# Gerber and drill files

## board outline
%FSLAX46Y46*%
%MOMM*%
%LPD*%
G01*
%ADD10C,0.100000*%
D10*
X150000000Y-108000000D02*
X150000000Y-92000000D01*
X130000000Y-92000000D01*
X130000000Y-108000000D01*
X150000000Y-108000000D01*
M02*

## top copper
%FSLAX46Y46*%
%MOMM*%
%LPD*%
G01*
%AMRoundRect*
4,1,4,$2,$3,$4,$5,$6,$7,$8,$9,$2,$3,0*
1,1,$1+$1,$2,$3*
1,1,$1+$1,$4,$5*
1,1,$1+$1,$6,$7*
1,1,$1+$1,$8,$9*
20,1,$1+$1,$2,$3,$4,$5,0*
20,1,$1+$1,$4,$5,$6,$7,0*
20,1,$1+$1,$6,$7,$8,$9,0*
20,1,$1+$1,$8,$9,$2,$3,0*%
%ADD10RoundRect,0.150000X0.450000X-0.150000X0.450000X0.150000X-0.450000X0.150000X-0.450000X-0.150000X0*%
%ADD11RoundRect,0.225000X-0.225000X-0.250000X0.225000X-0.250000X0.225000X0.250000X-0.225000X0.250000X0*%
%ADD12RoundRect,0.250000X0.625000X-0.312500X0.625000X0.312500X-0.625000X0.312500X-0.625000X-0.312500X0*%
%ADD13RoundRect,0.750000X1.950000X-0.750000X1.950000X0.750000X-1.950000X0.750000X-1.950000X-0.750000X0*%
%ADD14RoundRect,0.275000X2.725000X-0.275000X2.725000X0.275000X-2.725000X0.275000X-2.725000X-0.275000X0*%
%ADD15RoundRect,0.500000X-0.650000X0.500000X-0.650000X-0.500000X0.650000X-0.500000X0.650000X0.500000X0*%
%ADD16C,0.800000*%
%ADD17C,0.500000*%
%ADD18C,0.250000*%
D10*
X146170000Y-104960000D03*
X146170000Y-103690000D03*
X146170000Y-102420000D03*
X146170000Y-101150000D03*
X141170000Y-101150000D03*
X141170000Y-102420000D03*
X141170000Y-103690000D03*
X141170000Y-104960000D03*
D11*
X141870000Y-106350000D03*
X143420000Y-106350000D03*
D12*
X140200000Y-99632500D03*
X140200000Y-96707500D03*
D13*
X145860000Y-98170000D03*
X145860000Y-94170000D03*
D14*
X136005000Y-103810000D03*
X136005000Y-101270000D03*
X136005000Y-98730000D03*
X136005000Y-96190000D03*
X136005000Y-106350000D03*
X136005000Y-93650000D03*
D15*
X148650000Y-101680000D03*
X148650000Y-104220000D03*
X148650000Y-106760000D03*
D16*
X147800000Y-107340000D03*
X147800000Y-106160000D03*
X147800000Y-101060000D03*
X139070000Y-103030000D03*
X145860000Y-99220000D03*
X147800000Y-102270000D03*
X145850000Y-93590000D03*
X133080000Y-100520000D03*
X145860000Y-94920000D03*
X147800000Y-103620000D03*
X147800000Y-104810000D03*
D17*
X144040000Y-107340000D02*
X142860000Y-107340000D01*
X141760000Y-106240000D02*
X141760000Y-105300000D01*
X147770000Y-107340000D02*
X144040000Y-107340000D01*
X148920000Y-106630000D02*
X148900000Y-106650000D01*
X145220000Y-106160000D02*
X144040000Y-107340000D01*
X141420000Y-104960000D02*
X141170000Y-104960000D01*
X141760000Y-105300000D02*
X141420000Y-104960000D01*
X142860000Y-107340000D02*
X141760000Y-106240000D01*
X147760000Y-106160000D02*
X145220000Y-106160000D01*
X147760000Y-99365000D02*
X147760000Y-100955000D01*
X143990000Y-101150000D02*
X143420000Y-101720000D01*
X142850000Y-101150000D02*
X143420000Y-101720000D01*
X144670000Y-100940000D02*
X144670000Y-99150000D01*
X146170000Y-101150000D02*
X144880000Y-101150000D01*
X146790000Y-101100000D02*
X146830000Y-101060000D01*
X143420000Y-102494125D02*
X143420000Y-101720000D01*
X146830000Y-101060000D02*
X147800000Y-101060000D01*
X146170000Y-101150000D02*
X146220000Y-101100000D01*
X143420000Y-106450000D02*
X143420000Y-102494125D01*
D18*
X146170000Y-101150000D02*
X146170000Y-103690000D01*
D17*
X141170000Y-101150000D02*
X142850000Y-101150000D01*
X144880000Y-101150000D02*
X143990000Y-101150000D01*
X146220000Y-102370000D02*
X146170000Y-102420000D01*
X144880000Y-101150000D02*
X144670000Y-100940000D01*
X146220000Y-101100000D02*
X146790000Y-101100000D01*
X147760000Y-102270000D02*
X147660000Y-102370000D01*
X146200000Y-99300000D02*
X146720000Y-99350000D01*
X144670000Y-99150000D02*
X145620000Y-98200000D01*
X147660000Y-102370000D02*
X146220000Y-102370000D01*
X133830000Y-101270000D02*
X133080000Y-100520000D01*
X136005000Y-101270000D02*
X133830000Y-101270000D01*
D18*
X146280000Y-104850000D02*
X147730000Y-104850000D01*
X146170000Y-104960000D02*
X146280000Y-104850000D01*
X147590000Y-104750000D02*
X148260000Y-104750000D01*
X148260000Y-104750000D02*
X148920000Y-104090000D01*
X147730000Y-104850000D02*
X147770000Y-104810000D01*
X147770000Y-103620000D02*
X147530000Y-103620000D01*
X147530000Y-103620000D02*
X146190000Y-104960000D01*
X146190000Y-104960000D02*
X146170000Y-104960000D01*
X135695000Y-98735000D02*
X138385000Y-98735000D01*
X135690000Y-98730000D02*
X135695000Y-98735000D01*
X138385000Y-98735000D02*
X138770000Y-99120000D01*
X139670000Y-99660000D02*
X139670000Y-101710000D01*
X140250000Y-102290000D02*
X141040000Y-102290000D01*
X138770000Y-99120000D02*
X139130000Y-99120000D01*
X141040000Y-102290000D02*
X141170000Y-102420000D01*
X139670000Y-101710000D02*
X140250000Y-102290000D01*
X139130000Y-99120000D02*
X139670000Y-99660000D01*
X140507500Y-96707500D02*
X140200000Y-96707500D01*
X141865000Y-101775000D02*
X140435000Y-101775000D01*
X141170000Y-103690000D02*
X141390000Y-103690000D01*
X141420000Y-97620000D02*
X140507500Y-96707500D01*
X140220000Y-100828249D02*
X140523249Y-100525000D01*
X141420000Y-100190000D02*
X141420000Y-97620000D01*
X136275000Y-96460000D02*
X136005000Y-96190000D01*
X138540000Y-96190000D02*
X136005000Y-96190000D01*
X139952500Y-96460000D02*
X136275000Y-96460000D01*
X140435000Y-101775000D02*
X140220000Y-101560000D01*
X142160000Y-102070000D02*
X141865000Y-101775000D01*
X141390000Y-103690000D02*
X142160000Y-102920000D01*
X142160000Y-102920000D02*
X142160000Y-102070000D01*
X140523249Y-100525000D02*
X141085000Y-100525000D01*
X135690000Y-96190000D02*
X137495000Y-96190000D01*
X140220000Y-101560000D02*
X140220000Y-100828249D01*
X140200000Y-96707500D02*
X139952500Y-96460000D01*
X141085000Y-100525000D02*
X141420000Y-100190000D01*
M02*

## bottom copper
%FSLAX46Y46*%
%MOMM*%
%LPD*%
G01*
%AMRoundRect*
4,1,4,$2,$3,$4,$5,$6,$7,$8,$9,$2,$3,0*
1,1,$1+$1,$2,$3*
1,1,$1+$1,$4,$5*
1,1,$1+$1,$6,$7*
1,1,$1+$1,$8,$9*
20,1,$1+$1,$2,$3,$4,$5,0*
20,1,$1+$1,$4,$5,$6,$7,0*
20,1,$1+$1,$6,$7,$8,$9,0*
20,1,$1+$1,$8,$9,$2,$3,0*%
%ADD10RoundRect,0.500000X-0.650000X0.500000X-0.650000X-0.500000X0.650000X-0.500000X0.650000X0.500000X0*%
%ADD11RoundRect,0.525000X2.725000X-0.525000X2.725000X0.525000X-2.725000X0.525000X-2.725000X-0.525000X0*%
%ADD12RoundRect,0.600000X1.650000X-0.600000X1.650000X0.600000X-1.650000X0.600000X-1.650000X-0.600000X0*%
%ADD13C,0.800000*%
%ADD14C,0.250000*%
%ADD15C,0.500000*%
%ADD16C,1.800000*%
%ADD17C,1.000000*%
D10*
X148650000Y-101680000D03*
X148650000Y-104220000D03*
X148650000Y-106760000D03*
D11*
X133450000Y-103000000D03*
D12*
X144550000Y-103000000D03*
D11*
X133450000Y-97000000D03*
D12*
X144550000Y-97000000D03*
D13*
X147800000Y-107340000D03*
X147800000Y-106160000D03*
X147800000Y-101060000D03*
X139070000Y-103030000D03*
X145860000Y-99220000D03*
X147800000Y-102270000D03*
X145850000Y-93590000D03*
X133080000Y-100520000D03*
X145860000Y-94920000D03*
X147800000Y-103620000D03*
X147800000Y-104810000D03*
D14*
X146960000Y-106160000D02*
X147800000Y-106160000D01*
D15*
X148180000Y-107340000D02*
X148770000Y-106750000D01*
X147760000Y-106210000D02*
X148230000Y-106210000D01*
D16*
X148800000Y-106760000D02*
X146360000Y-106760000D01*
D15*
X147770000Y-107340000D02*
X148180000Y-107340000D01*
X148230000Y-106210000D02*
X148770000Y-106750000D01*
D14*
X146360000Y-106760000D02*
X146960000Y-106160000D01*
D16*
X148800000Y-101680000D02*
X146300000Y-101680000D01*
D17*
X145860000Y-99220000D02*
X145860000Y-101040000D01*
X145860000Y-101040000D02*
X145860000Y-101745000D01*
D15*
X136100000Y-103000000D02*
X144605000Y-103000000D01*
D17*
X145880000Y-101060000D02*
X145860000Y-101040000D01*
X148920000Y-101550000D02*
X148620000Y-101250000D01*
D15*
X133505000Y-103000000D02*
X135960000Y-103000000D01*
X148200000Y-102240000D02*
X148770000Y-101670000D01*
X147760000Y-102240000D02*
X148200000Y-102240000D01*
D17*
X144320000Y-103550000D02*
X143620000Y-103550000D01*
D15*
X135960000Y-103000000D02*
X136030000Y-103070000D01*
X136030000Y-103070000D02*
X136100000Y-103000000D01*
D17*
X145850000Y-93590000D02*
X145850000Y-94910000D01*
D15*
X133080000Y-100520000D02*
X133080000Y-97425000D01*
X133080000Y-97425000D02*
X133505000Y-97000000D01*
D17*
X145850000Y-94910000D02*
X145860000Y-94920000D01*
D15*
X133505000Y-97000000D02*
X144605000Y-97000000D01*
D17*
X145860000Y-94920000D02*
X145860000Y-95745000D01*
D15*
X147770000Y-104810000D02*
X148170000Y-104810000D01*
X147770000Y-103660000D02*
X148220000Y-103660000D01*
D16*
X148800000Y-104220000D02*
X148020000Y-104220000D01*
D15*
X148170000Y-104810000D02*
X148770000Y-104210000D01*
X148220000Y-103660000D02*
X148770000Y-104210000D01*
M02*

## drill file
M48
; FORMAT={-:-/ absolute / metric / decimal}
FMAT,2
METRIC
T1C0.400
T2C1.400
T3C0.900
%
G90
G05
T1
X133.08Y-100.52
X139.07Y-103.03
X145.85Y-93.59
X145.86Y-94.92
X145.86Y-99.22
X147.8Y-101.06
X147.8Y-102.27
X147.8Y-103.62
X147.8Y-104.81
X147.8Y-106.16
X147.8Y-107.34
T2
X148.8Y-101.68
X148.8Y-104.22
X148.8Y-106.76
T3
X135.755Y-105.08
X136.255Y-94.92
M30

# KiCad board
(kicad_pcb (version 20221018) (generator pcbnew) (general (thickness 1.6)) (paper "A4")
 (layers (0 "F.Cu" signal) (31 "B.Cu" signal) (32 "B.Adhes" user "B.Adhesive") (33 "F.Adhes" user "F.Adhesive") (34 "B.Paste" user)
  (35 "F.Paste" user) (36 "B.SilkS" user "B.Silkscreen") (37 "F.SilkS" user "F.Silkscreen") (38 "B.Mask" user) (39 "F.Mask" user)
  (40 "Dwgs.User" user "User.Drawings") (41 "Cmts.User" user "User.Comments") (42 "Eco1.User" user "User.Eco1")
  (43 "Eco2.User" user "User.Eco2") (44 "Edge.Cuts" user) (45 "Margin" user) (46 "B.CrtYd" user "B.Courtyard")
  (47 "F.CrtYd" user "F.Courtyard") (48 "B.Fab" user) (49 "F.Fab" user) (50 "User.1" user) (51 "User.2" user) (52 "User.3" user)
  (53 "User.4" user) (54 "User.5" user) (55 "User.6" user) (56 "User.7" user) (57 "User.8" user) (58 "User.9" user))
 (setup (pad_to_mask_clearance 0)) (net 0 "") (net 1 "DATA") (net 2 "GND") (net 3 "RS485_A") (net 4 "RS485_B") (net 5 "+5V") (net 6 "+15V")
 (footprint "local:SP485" (layer "F.Cu") (at 143.67 103.055 90)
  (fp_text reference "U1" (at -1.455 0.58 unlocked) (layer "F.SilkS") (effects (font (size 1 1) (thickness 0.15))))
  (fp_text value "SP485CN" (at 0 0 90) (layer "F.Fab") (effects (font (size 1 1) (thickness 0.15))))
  (pad "1" smd roundrect (at -1.905 2.5 90) (size 0.6 1.2) (layers "F.Cu" "F.Paste" "F.Mask") (roundrect_rratio 0.25) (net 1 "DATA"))
  (pad "2" smd roundrect (at -0.635 2.5 90) (size 0.6 1.2) (layers "F.Cu" "F.Paste" "F.Mask") (roundrect_rratio 0.25) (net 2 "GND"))
  (pad "3" smd roundrect (at 0.635 2.5 90) (size 0.6 1.2) (layers "F.Cu" "F.Paste" "F.Mask") (roundrect_rratio 0.25) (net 2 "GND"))
  (pad "4" smd roundrect (at 1.905 2.5 90) (size 0.6 1.2) (layers "F.Cu" "F.Paste" "F.Mask") (roundrect_rratio 0.25) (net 2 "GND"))
  (pad "5" smd roundrect (at 1.905 -2.5 90) (size 0.6 1.2) (layers "F.Cu" "F.Paste" "F.Mask") (roundrect_rratio 0.25) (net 2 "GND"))
  (pad "6" smd roundrect (at 0.635 -2.5 90) (size 0.6 1.2) (layers "F.Cu" "F.Paste" "F.Mask") (roundrect_rratio 0.25) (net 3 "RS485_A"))
  (pad "7" smd roundrect (at -0.635 -2.5 90) (size 0.6 1.2) (layers "F.Cu" "F.Paste" "F.Mask") (roundrect_rratio 0.25) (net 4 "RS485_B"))
  (pad "8" smd roundrect (at -1.905 -2.5 90) (size 0.6 1.2) (layers "F.Cu" "F.Paste" "F.Mask") (roundrect_rratio 0.25) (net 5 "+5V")))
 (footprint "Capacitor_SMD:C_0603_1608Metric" (layer "F.Cu") (at 142.645 106.35)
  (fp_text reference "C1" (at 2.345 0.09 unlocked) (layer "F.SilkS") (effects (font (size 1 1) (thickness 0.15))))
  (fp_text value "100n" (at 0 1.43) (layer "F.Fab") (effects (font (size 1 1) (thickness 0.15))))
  (pad "1" smd roundrect (at -0.775 0) (size 0.9 0.95) (layers "F.Cu" "F.Paste" "F.Mask") (roundrect_rratio 0.25) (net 5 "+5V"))
  (pad "2" smd roundrect (at 0.775 0) (size 0.9 0.95) (layers "F.Cu" "F.Paste" "F.Mask") (roundrect_rratio 0.25) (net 2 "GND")))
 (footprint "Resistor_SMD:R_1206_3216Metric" (layer "F.Cu") (at 140.2 98.17 90)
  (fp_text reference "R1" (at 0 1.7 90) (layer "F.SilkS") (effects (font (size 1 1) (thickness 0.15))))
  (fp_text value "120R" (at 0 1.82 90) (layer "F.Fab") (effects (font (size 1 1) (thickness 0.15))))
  (pad "1" smd roundrect (at -1.4625 0 90) (size 1.125 1.75) (layers "F.Cu" "F.Paste" "F.Mask") (roundrect_rratio 0.222222)
   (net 3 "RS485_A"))
  (pad "2" smd roundrect (at 1.4625 0 90) (size 1.125 1.75) (layers "F.Cu" "F.Paste" "F.Mask") (roundrect_rratio 0.222222) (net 4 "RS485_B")))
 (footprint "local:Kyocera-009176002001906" (layer "F.Cu") (at 145.86 96.17 90)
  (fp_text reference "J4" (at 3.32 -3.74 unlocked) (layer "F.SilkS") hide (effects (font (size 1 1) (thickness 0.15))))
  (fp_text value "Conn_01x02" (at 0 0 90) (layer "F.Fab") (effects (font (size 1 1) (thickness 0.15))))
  (pad "1" smd roundrect (at -2 0 90) (size 3 5.4) (layers "F.Cu" "F.Paste" "F.Mask") (roundrect_rratio 0.25) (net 2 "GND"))
  (pad "2" smd roundrect (at 2 0 90) (size 3 5.4) (layers "F.Cu" "F.Paste" "F.Mask") (roundrect_rratio 0.25) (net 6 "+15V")))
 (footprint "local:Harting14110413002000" (layer "F.Cu") (at 136.005 100 90)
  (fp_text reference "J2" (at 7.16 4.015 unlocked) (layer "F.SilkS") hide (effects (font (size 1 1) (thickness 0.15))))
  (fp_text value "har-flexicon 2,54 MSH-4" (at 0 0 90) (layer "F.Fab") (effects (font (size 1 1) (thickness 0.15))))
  (pad "" np_thru_hole circle (at -5.08 -0.25 90) (size 0.9 0.9) (drill 0.9) (layers "*.Cu" "*.Mask"))
  (pad "" np_thru_hole circle (at 5.08 0.25 90) (size 0.9 0.9) (drill 0.9) (layers "*.Cu" "*.Mask"))
  (pad "1" smd roundrect (at -3.81 0 90) (size 1.1 6) (layers "F.Cu" "F.Paste" "F.Mask") (roundrect_rratio 0.25) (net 2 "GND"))
  (pad "2" smd roundrect (at -1.27 0 90) (size 1.1 6) (layers "F.Cu" "F.Paste" "F.Mask") (roundrect_rratio 0.25) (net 6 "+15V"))
  (pad "3" smd roundrect (at 1.27 0 90) (size 1.1 6) (layers "F.Cu" "F.Paste" "F.Mask") (roundrect_rratio 0.25) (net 3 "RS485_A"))
  (pad "4" smd roundrect (at 3.81 0 90) (size 1.1 6) (layers "F.Cu" "F.Paste" "F.Mask") (roundrect_rratio 0.25) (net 4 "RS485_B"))
  (pad "MP1" smd roundrect (at -6.35 0 90) (size 1.1 6) (layers "F.Cu" "F.Paste" "F.Mask") (roundrect_rratio 0.25))
  (pad "MP2" smd roundrect (at 6.35 0 90) (size 1.1 6) (layers "F.Cu" "F.Paste" "F.Mask") (roundrect_rratio 0.25)))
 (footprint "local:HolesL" (layer "F.Cu") (at 148.8 104.22 -90)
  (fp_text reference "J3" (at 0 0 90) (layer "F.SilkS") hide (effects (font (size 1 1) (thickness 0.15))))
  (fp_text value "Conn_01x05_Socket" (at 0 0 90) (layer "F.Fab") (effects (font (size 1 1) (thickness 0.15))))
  (pad "1" thru_hole roundrect (at -2.54 0 270) (size 2 2.3) (drill 1.4 (offset 0 0.15)) (layers "*.Cu" "*.Mask") (roundrect_rratio 0.25)
   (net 2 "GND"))
  (pad "2" thru_hole roundrect (at 0 0 270) (size 2 2.3) (drill 1.4 (offset 0 0.15)) (layers "*.Cu" "*.Mask") (roundrect_rratio 0.25)
   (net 1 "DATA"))
  (pad "3" thru_hole roundrect (at 2.54 0 270) (size 2 2.3) (drill 1.4 (offset 0 0.15)) (layers "*.Cu" "*.Mask") (roundrect_rratio 0.25)
   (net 5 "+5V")))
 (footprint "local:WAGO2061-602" (layer "B.Cu") (at 138.2 100 90)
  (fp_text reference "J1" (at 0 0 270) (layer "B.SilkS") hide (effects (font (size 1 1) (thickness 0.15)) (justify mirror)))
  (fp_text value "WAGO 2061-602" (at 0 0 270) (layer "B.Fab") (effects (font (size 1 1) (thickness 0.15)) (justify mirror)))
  (pad "1" smd roundrect (at -3 -4.75 90) (size 2.1 6.5) (layers "B.Cu" "B.Paste" "B.Mask") (roundrect_rratio 0.25) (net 2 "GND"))
  (pad "1" smd roundrect (at -3 6.35 90) (size 2.4 4.5) (layers "B.Cu" "B.Paste" "B.Mask") (roundrect_rratio 0.25) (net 2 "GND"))
  (pad "2" smd roundrect (at 3 -4.75 90) (size 2.1 6.5) (layers "B.Cu" "B.Paste" "B.Mask") (roundrect_rratio 0.25) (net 6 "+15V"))
  (pad "2" smd roundrect (at 3 6.35 90) (size 2.4 4.5) (layers "B.Cu" "B.Paste" "B.Mask") (roundrect_rratio 0.25) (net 6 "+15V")))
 (gr_poly (pts (xy 150 108) (xy 150 92) (xy 130 92) (xy 130 108)) (stroke (width 0.1) (type solid)) (fill none) (layer "Edge.Cuts"))
 (segment (start 144.04 107.34) (end 142.86 107.34) (width 0.5) (layer "F.Cu") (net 5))
 (segment (start 141.76 106.24) (end 141.76 105.3) (width 0.5) (layer "F.Cu") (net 5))
 (segment (start 147.77 107.34) (end 144.04 107.34) (width 0.5) (layer "F.Cu") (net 5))
 (segment (start 148.92 106.63) (end 148.9 106.65) (width 0.5) (layer "F.Cu") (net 5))
 (segment (start 145.22 106.16) (end 144.04 107.34) (width 0.5) (layer "F.Cu") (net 5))
 (segment (start 141.42 104.96) (end 141.17 104.96) (width 0.5) (layer "F.Cu") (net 5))
 (segment (start 141.76 105.3) (end 141.42 104.96) (width 0.5) (layer "F.Cu") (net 5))
 (segment (start 142.86 107.34) (end 141.76 106.24) (width 0.5) (layer "F.Cu") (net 5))
 (segment (start 147.76 106.16) (end 145.22 106.16) (width 0.5) (layer "F.Cu") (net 5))
 (via (at 147.8 107.34) (size 0.8) (drill 0.4) (layers "F.Cu" "B.Cu") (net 5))
 (via (at 147.8 106.16) (size 0.8) (drill 0.4) (layers "F.Cu" "B.Cu") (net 5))
 (segment (start 146.96 106.16) (end 147.8 106.16) (width 0.25) (layer "B.Cu") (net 5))
 (segment (start 148.18 107.34) (end 148.77 106.75) (width 0.5) (layer "B.Cu") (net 5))
 (segment (start 147.76 106.21) (end 148.23 106.21) (width 0.5) (layer "B.Cu") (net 5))
 (segment (start 148.8 106.76) (end 146.36 106.76) (width 1.8) (layer "B.Cu") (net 5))
 (segment (start 147.77 107.34) (end 148.18 107.34) (width 0.5) (layer "B.Cu") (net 5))
 (segment (start 148.23 106.21) (end 148.77 106.75) (width 0.5) (layer "B.Cu") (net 5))
 (segment (start 146.36 106.76) (end 146.96 106.16) (width 0.25) (layer "B.Cu") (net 5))
 (segment (start 147.76 99.365) (end 147.76 100.955) (width 0.5) (layer "F.Cu") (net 2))
 (segment (start 143.99 101.15) (end 143.42 101.72) (width 0.5) (layer "F.Cu") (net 2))
 (segment (start 142.85 101.15) (end 143.42 101.72) (width 0.5) (layer "F.Cu") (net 2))
 (segment (start 144.67 100.94) (end 144.67 99.15) (width 0.5) (layer "F.Cu") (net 2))
 (segment (start 146.17 101.15) (end 144.88 101.15) (width 0.5) (layer "F.Cu") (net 2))
 (segment (start 146.79 101.1) (end 146.83 101.06) (width 0.5) (layer "F.Cu") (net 2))
 (segment (start 143.42 102.494125) (end 143.42 101.72) (width 0.5) (layer "F.Cu") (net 2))
 (segment (start 146.83 101.06) (end 147.8 101.06) (width 0.5) (layer "F.Cu") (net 2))
 (segment (start 146.17 101.15) (end 146.22 101.1) (width 0.5) (layer "F.Cu") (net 2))
 (segment (start 143.42 106.45) (end 143.42 102.494125) (width 0.5) (layer "F.Cu") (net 2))
 (segment (start 146.17 101.15) (end 146.17 103.69) (width 0.25) (layer "F.Cu") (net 2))
 (segment (start 141.17 101.15) (end 142.85 101.15) (width 0.5) (layer "F.Cu") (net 2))
 (segment (start 144.88 101.15) (end 143.99 101.15) (width 0.5) (layer "F.Cu") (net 2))
 (segment (start 146.22 102.37) (end 146.17 102.42) (width 0.5) (layer "F.Cu") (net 2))
 (segment (start 144.88 101.15) (end 144.67 100.94) (width 0.5) (layer "F.Cu") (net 2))
 (segment (start 146.22 101.1) (end 146.79 101.1) (width 0.5) (layer "F.Cu") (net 2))
 (segment (start 147.76 102.27) (end 147.66 102.37) (width 0.5) (layer "F.Cu") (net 2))
 (segment (start 146.2 99.3) (end 146.72 99.35) (width 0.5) (layer "F.Cu") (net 2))
 (segment (start 144.67 99.15) (end 145.62 98.2) (width 0.5) (layer "F.Cu") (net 2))
 (segment (start 147.66 102.37) (end 146.22 102.37) (width 0.5) (layer "F.Cu") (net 2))
 (via (at 147.8 101.06) (size 0.8) (drill 0.4) (layers "F.Cu" "B.Cu") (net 2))
 (via (at 139.07 103.03) (size 0.8) (drill 0.4) (layers "F.Cu" "B.Cu") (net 2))
 (via (at 145.86 99.22) (size 0.8) (drill 0.4) (layers "F.Cu" "B.Cu") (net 2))
 (via (at 147.8 102.27) (size 0.8) (drill 0.4) (layers "F.Cu" "B.Cu") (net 2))
 (segment (start 148.8 101.68) (end 146.3 101.68) (width 1.8) (layer "B.Cu") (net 2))
 (segment (start 145.86 99.22) (end 145.86 101.04) (width 1) (layer "B.Cu") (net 2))
 (segment (start 145.86 101.04) (end 145.86 101.745) (width 1) (layer "B.Cu") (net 2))
 (segment (start 136.1 103) (end 144.605 103) (width 0.5) (layer "B.Cu") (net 2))
 (segment (start 145.88 101.06) (end 145.86 101.04) (width 1) (layer "B.Cu") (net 2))
 (segment (start 148.92 101.55) (end 148.62 101.25) (width 1) (layer "B.Cu") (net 2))
 (segment (start 133.505 103) (end 135.96 103) (width 0.5) (layer "B.Cu") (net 2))
 (segment (start 148.2 102.24) (end 148.77 101.67) (width 0.5) (layer "B.Cu") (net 2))
 (segment (start 147.76 102.24) (end 148.2 102.24) (width 0.5) (layer "B.Cu") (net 2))
 (segment (start 144.32 103.55) (end 143.62 103.55) (width 1) (layer "B.Cu") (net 2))
 (segment (start 135.96 103) (end 136.03 103.07) (width 0.5) (layer "B.Cu") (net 2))
 (segment (start 136.03 103.07) (end 136.1 103) (width 0.5) (layer "B.Cu") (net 2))
 (segment (start 133.83 101.27) (end 133.08 100.52) (width 0.5) (layer "F.Cu") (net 6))
 (segment (start 136.005 101.27) (end 133.83 101.27) (width 0.5) (layer "F.Cu") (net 6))
 (via (at 145.85 93.59) (size 0.8) (drill 0.4) (layers "F.Cu" "B.Cu") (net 6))
 (via (at 133.08 100.52) (size 0.8) (drill 0.4) (layers "F.Cu" "B.Cu") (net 6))
 (via (at 145.86 94.92) (size 0.8) (drill 0.4) (layers "F.Cu" "B.Cu") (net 6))
 (segment (start 145.85 93.59) (end 145.85 94.91) (width 1) (layer "B.Cu") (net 6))
 (segment (start 133.08 100.52) (end 133.08 97.425) (width 0.5) (layer "B.Cu") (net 6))
 (segment (start 133.08 97.425) (end 133.505 97) (width 0.5) (layer "B.Cu") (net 6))
 (segment (start 145.85 94.91) (end 145.86 94.92) (width 1) (layer "B.Cu") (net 6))
 (segment (start 133.505 97) (end 144.605 97) (width 0.5) (layer "B.Cu") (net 6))
 (segment (start 145.86 94.92) (end 145.86 95.745) (width 1) (layer "B.Cu") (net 6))
 (segment (start 146.28 104.85) (end 147.73 104.85) (width 0.25) (layer "F.Cu") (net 1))
 (segment (start 146.17 104.96) (end 146.28 104.85) (width 0.25) (layer "F.Cu") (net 1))
 (segment (start 147.59 104.75) (end 148.26 104.75) (width 0.25) (layer "F.Cu") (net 1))
 (segment (start 148.26 104.75) (end 148.92 104.09) (width 0.25) (layer "F.Cu") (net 1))
 (segment (start 147.73 104.85) (end 147.77 104.81) (width 0.25) (layer "F.Cu") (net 1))
 (segment (start 147.77 103.62) (end 147.53 103.62) (width 0.25) (layer "F.Cu") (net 1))
 (segment (start 147.53 103.62) (end 146.19 104.96) (width 0.25) (layer "F.Cu") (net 1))
 (segment (start 146.19 104.96) (end 146.17 104.96) (width 0.25) (layer "F.Cu") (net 1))
 (via (at 147.8 103.62) (size 0.8) (drill 0.4) (layers "F.Cu" "B.Cu") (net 1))
 (via (at 147.8 104.81) (size 0.8) (drill 0.4) (layers "F.Cu" "B.Cu") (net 1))
 (segment (start 147.77 104.81) (end 148.17 104.81) (width 0.5) (layer "B.Cu") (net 1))
 (segment (start 147.77 103.66) (end 148.22 103.66) (width 0.5) (layer "B.Cu") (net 1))
 (segment (start 148.8 104.22) (end 148.02 104.22) (width 1.8) (layer "B.Cu") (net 1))
 (segment (start 148.17 104.81) (end 148.77 104.21) (width 0.5) (layer "B.Cu") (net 1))
 (segment (start 148.22 103.66) (end 148.77 104.21) (width 0.5) (layer "B.Cu") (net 1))
 (segment (start 135.695 98.735) (end 138.385 98.735) (width 0.25) (layer "F.Cu") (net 3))
 (segment (start 135.69 98.73) (end 135.695 98.735) (width 0.25) (layer "F.Cu") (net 3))
 (segment (start 138.385 98.735) (end 138.77 99.12) (width 0.25) (layer "F.Cu") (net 3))
 (segment (start 139.67 99.66) (end 139.67 101.71) (width 0.25) (layer "F.Cu") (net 3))
 (segment (start 140.25 102.29) (end 141.04 102.29) (width 0.25) (layer "F.Cu") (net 3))
 (segment (start 138.77 99.12) (end 139.13 99.12) (width 0.25) (layer "F.Cu") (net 3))
 (segment (start 141.04 102.29) (end 141.17 102.42) (width 0.25) (layer "F.Cu") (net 3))
 (segment (start 139.67 101.71) (end 140.25 102.29) (width 0.25) (layer "F.Cu") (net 3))
 (segment (start 139.13 99.12) (end 139.67 99.66) (width 0.25) (layer "F.Cu") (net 3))
 (segment (start 140.5075 96.7075) (end 140.2 96.7075) (width 0.25) (layer "F.Cu") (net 4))
 (segment (start 141.865 101.775) (end 140.435 101.775) (width 0.25) (layer "F.Cu") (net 4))
 (segment (start 141.17 103.69) (end 141.39 103.69) (width 0.25) (layer "F.Cu") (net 4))
 (segment (start 141.42 97.62) (end 140.5075 96.7075) (width 0.25) (layer "F.Cu") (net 4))
 (segment (start 140.22 100.828249) (end 140.523249 100.525) (width 0.25) (layer "F.Cu") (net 4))
 (segment (start 141.42 100.19) (end 141.42 97.62) (width 0.25) (layer "F.Cu") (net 4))
 (segment (start 136.275 96.46) (end 136.005 96.19) (width 0.25) (layer "F.Cu") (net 4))
 (segment (start 138.54 96.19) (end 136.005 96.19) (width 0.25) (layer "F.Cu") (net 4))
 (segment (start 139.9525 96.46) (end 136.275 96.46) (width 0.25) (layer "F.Cu") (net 4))
 (segment (start 140.435 101.775) (end 140.22 101.56) (width 0.25) (layer "F.Cu") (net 4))
 (segment (start 142.16 102.07) (end 141.865 101.775) (width 0.25) (layer "F.Cu") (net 4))
 (segment (start 141.39 103.69) (end 142.16 102.92) (width 0.25) (layer "F.Cu") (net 4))
 (segment (start 142.16 102.92) (end 142.16 102.07) (width 0.25) (layer "F.Cu") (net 4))
 (segment (start 140.523249 100.525) (end 141.085 100.525) (width 0.25) (layer "F.Cu") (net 4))
 (segment (start 135.69 96.19) (end 137.495 96.19) (width 0.25) (layer "F.Cu") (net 4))
 (segment (start 140.22 101.56) (end 140.22 100.828249) (width 0.25) (layer "F.Cu") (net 4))
 (segment (start 140.2 96.7075) (end 139.9525 96.46) (width 0.25) (layer "F.Cu") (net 4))
 (segment (start 141.085 100.525) (end 141.42 100.19) (width 0.25) (layer "F.Cu") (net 4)))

